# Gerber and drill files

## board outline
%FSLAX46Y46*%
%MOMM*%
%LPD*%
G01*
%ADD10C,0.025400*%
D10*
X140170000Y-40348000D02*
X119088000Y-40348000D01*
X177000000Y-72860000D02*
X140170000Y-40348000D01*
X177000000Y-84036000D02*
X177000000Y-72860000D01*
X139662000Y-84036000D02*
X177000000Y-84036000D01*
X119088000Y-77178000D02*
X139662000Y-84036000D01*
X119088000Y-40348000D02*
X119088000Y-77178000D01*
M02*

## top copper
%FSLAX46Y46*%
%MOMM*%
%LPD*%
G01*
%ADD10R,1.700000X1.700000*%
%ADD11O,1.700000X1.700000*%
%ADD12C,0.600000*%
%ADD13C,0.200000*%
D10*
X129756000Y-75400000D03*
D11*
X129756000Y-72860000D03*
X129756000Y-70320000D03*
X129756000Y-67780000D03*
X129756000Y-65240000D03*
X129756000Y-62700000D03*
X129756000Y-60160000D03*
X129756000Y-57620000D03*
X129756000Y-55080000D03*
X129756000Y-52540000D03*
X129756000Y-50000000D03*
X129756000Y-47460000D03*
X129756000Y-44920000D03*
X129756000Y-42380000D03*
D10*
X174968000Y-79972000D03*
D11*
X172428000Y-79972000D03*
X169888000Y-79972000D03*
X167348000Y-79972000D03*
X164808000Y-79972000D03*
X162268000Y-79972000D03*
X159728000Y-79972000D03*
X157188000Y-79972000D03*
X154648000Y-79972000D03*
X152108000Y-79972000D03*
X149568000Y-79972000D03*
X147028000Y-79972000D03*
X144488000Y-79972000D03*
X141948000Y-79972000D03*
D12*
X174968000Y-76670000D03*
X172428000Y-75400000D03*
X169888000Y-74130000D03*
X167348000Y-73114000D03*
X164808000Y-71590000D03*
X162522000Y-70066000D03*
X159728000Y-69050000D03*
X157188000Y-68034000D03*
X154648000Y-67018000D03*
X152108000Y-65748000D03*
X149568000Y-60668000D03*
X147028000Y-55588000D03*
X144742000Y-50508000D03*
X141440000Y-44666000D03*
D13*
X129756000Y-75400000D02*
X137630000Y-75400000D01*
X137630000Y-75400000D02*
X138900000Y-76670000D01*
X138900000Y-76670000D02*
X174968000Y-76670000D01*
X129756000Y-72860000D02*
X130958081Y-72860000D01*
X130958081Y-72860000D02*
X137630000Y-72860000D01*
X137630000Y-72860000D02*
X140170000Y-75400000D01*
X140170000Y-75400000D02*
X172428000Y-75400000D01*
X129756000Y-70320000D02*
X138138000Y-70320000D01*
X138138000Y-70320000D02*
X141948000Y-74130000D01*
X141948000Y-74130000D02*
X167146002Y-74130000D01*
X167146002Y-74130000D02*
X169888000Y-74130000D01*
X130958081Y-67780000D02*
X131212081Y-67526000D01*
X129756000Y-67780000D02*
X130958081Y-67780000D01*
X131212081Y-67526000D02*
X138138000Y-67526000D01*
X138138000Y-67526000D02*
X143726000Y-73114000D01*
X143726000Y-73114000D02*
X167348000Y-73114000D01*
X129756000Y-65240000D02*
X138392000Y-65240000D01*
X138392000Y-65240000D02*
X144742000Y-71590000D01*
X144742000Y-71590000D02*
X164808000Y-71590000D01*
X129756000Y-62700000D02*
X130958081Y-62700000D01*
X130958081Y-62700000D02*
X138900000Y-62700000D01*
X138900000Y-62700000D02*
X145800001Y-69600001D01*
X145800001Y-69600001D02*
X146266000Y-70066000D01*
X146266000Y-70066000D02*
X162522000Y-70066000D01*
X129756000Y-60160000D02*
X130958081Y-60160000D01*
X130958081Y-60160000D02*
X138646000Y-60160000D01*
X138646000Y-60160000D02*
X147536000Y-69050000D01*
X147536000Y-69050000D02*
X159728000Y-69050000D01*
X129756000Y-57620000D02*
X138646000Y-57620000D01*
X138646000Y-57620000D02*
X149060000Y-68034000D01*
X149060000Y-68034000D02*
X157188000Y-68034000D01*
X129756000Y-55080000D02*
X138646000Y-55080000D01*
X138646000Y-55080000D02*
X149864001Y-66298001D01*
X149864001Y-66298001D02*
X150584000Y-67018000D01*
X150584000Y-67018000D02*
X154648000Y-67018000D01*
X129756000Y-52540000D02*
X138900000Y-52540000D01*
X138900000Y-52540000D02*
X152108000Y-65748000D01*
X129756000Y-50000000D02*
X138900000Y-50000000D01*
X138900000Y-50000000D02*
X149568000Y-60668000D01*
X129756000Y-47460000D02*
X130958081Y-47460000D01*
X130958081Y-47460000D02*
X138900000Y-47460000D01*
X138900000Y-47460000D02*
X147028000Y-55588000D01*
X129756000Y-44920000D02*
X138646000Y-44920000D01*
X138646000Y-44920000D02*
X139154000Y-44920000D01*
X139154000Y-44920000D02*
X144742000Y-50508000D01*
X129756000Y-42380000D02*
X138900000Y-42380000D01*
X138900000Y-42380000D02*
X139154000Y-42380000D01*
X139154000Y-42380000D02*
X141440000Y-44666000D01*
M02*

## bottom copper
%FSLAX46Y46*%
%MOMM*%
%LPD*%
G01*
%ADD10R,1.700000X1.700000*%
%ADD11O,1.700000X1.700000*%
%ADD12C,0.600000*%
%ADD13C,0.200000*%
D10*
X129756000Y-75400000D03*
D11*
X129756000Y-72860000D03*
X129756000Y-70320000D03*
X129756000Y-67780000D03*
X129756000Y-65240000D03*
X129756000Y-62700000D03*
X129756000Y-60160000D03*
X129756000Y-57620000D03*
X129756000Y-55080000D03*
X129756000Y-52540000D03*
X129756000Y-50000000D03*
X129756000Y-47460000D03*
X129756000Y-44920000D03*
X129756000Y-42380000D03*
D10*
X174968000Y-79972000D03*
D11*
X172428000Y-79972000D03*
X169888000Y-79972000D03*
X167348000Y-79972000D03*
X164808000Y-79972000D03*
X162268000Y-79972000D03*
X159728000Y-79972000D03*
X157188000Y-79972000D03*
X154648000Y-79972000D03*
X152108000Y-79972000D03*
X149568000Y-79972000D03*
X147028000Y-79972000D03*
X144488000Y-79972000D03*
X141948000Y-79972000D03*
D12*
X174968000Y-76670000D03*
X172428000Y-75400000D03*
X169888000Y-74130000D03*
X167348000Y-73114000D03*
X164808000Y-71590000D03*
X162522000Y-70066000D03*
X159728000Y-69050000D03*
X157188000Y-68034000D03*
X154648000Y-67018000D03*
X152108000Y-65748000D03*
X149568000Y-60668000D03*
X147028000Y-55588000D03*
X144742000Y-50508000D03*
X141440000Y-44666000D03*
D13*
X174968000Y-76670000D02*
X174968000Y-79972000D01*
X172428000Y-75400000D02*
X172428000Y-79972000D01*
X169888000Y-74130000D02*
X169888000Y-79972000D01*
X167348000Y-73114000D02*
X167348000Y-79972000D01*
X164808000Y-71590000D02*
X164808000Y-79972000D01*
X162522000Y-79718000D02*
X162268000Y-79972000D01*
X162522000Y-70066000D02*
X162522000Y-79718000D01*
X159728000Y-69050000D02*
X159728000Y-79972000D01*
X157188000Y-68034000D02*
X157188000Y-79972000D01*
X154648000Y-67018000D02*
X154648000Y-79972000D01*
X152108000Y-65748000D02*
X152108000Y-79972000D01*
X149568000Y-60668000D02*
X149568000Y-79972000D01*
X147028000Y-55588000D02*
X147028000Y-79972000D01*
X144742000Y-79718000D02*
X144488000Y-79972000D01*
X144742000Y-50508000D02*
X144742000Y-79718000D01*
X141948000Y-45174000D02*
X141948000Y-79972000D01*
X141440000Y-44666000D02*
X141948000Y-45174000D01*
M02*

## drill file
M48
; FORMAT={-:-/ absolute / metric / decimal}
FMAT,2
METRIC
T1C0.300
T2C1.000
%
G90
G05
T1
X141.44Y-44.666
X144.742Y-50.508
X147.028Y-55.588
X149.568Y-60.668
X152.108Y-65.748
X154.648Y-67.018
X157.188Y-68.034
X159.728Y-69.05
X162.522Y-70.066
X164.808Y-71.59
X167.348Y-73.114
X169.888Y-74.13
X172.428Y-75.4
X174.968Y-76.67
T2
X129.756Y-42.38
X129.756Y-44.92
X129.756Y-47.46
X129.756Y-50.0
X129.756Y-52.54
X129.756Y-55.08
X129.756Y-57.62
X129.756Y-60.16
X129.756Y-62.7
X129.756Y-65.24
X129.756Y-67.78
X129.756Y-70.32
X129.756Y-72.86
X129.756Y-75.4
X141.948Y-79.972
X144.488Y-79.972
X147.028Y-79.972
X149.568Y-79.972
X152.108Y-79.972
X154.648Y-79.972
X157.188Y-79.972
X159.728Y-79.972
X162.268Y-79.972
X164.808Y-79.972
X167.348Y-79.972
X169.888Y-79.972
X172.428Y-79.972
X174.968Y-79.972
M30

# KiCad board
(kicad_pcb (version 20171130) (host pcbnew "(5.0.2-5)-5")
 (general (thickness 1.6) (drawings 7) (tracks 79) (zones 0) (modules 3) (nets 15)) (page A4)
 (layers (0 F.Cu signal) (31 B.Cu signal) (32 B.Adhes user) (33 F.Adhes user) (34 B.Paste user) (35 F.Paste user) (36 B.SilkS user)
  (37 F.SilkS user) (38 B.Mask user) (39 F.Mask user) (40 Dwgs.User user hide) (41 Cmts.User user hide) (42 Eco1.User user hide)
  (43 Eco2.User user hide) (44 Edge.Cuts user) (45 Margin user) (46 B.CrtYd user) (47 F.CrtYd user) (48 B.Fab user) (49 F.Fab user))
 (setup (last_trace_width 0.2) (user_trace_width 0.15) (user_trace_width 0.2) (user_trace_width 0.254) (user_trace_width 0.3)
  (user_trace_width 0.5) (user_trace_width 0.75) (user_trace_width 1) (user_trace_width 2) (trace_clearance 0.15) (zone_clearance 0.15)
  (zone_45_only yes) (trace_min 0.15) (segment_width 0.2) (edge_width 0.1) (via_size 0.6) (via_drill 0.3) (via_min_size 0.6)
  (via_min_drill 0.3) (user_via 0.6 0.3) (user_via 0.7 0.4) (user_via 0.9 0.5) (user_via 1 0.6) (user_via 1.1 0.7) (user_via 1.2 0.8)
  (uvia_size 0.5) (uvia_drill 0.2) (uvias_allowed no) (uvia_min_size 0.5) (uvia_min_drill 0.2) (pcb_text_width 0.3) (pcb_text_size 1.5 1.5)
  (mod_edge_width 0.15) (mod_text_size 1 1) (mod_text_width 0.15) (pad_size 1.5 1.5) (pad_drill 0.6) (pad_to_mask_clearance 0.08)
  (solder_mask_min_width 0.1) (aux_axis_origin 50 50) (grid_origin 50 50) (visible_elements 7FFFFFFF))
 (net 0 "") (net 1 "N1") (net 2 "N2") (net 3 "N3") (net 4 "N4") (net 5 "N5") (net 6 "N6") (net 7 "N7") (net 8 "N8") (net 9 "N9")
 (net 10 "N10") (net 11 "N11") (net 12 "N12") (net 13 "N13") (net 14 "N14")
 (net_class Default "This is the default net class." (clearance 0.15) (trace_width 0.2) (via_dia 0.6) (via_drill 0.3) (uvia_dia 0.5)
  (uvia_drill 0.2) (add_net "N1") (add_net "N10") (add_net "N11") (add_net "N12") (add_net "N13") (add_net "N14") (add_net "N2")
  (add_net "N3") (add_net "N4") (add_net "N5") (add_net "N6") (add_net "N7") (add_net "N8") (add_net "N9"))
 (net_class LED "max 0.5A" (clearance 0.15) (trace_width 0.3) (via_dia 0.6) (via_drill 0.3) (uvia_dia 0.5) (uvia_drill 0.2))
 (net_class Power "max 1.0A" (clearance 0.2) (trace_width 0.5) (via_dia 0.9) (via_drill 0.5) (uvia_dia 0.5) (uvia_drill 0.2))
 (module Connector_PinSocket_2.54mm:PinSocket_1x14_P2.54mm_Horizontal (layer B.Cu) (at 129.756 75.4)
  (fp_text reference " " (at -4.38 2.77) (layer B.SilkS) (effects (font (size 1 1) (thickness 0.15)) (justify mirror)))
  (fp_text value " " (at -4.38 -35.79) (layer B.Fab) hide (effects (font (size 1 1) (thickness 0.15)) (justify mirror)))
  (pad 1 thru_hole rect (at 0 0) (size 1.7 1.7) (drill 1) (layers *.Cu *.Mask) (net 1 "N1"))
  (pad 2 thru_hole oval (at 0 -2.54) (size 1.7 1.7) (drill 1) (layers *.Cu *.Mask) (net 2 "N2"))
  (pad 3 thru_hole oval (at 0 -5.08) (size 1.7 1.7) (drill 1) (layers *.Cu *.Mask) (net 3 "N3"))
  (pad 4 thru_hole oval (at 0 -7.62) (size 1.7 1.7) (drill 1) (layers *.Cu *.Mask) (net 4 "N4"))
  (pad 5 thru_hole oval (at 0 -10.16) (size 1.7 1.7) (drill 1) (layers *.Cu *.Mask) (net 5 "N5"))
  (pad 6 thru_hole oval (at 0 -12.7) (size 1.7 1.7) (drill 1) (layers *.Cu *.Mask) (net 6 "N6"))
  (pad 7 thru_hole oval (at 0 -15.24) (size 1.7 1.7) (drill 1) (layers *.Cu *.Mask) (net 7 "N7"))
  (pad 8 thru_hole oval (at 0 -17.78) (size 1.7 1.7) (drill 1) (layers *.Cu *.Mask) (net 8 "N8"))
  (pad 9 thru_hole oval (at 0 -20.32) (size 1.7 1.7) (drill 1) (layers *.Cu *.Mask) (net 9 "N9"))
  (pad 10 thru_hole oval (at 0 -22.86) (size 1.7 1.7) (drill 1) (layers *.Cu *.Mask) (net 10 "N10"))
  (pad 11 thru_hole oval (at 0 -25.4) (size 1.7 1.7) (drill 1) (layers *.Cu *.Mask) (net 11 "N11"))
  (pad 12 thru_hole oval (at 0 -27.94) (size 1.7 1.7) (drill 1) (layers *.Cu *.Mask) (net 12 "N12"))
  (pad 13 thru_hole oval (at 0 -30.48) (size 1.7 1.7) (drill 1) (layers *.Cu *.Mask) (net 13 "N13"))
  (pad 14 thru_hole oval (at 0 -33.02) (size 1.7 1.7) (drill 1) (layers *.Cu *.Mask) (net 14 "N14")))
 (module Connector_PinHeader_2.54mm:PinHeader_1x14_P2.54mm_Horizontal (layer F.Cu) (at 174.968 79.972 270)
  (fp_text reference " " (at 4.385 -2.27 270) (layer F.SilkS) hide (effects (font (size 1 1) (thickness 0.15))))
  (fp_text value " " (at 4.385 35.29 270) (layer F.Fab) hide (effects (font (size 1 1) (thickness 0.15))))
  (pad 1 thru_hole rect (at 0 0 270) (size 1.7 1.7) (drill 1) (layers *.Cu *.Mask) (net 1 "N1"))
  (pad 2 thru_hole oval (at 0 2.54 270) (size 1.7 1.7) (drill 1) (layers *.Cu *.Mask) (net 2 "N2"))
  (pad 3 thru_hole oval (at 0 5.08 270) (size 1.7 1.7) (drill 1) (layers *.Cu *.Mask) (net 3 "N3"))
  (pad 4 thru_hole oval (at 0 7.62 270) (size 1.7 1.7) (drill 1) (layers *.Cu *.Mask) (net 4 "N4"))
  (pad 5 thru_hole oval (at 0 10.16 270) (size 1.7 1.7) (drill 1) (layers *.Cu *.Mask) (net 5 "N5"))
  (pad 6 thru_hole oval (at 0 12.7 270) (size 1.7 1.7) (drill 1) (layers *.Cu *.Mask) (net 6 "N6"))
  (pad 7 thru_hole oval (at 0 15.24 270) (size 1.7 1.7) (drill 1) (layers *.Cu *.Mask) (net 7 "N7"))
  (pad 8 thru_hole oval (at 0 17.78 270) (size 1.7 1.7) (drill 1) (layers *.Cu *.Mask) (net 8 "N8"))
  (pad 9 thru_hole oval (at 0 20.32 270) (size 1.7 1.7) (drill 1) (layers *.Cu *.Mask) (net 9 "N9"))
  (pad 10 thru_hole oval (at 0 22.86 270) (size 1.7 1.7) (drill 1) (layers *.Cu *.Mask) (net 10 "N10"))
  (pad 11 thru_hole oval (at 0 25.4 270) (size 1.7 1.7) (drill 1) (layers *.Cu *.Mask) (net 11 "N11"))
  (pad 12 thru_hole oval (at 0 27.94 270) (size 1.7 1.7) (drill 1) (layers *.Cu *.Mask) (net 12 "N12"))
  (pad 13 thru_hole oval (at 0 30.48 270) (size 1.7 1.7) (drill 1) (layers *.Cu *.Mask) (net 13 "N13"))
  (pad 14 thru_hole oval (at 0 33.02 270) (size 1.7 1.7) (drill 1) (layers *.Cu *.Mask) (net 14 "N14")))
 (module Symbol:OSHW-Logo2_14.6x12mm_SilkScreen (layer B.Cu) (at 152.108 66.256 180)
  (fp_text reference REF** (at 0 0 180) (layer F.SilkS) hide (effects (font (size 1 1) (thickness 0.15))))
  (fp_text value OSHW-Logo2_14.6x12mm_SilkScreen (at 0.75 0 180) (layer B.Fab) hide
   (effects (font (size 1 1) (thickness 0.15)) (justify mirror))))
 (gr_line (start 140.17 40.348) (end 119.088 40.348) (layer Edge.Cuts) (width 0.0254))
 (gr_line (start 177 72.86) (end 140.17 40.348) (layer Edge.Cuts) (width 0.0254))
 (gr_line (start 177 84.036) (end 177 72.86) (layer Edge.Cuts) (width 0.0254))
 (gr_line (start 139.662 84.036) (end 177 84.036) (layer Edge.Cuts) (width 0.0254))
 (gr_line (start 119.088 77.178) (end 139.662 84.036) (layer Edge.Cuts) (width 0.0254))
 (gr_line (start 119.088 40.348) (end 119.088 77.178) (layer Edge.Cuts) (width 0.0254))
 (segment (start 129.756 75.4) (end 137.63 75.4) (width 0.2) (layer F.Cu) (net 1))
 (segment (start 137.63 75.4) (end 138.9 76.67) (width 0.2) (layer F.Cu) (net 1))
 (segment (start 138.9 76.67) (end 174.968 76.67) (width 0.2) (layer F.Cu) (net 1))
 (via (at 174.968 76.67) (size 0.6) (drill 0.3) (layers F.Cu B.Cu) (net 1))
 (segment (start 174.968 76.67) (end 174.968 79.972) (width 0.2) (layer B.Cu) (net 1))
 (segment (start 129.756 72.86) (end 130.958081 72.86) (width 0.2) (layer F.Cu) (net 2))
 (segment (start 130.958081 72.86) (end 137.63 72.86) (width 0.2) (layer F.Cu) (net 2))
 (segment (start 137.63 72.86) (end 140.17 75.4) (width 0.2) (layer F.Cu) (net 2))
 (segment (start 140.17 75.4) (end 172.428 75.4) (width 0.2) (layer F.Cu) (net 2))
 (via (at 172.428 75.4) (size 0.6) (drill 0.3) (layers F.Cu B.Cu) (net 2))
 (segment (start 172.428 75.4) (end 172.428 79.972) (width 0.2) (layer B.Cu) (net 2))
 (segment (start 129.756 70.32) (end 138.138 70.32) (width 0.2) (layer F.Cu) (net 3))
 (segment (start 138.138 70.32) (end 141.948 74.13) (width 0.2) (layer F.Cu) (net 3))
 (segment (start 141.948 74.13) (end 167.146002 74.13) (width 0.2) (layer F.Cu) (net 3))
 (via (at 169.888 74.13) (size 0.6) (drill 0.3) (layers F.Cu B.Cu) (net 3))
 (segment (start 167.146002 74.13) (end 169.888 74.13) (width 0.2) (layer F.Cu) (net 3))
 (segment (start 169.888 74.13) (end 169.888 79.972) (width 0.2) (layer B.Cu) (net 3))
 (segment (start 130.958081 67.78) (end 131.212081 67.526) (width 0.2) (layer F.Cu) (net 4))
 (segment (start 129.756 67.78) (end 130.958081 67.78) (width 0.2) (layer F.Cu) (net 4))
 (segment (start 131.212081 67.526) (end 138.138 67.526) (width 0.2) (layer F.Cu) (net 4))
 (segment (start 138.138 67.526) (end 143.726 73.114) (width 0.2) (layer F.Cu) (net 4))
 (via (at 167.348 73.114) (size 0.6) (drill 0.3) (layers F.Cu B.Cu) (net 4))
 (segment (start 143.726 73.114) (end 167.348 73.114) (width 0.2) (layer F.Cu) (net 4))
 (segment (start 167.348 73.114) (end 167.348 79.972) (width 0.2) (layer B.Cu) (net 4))
 (segment (start 129.756 65.24) (end 138.392 65.24) (width 0.2) (layer F.Cu) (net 5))
 (segment (start 138.392 65.24) (end 144.742 71.59) (width 0.2) (layer F.Cu) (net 5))
 (segment (start 144.742 71.59) (end 164.808 71.59) (width 0.2) (layer F.Cu) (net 5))
 (via (at 164.808 71.59) (size 0.6) (drill 0.3) (layers F.Cu B.Cu) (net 5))
 (segment (start 164.808 71.59) (end 164.808 79.972) (width 0.2) (layer B.Cu) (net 5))
 (segment (start 129.756 62.7) (end 130.958081 62.7) (width 0.2) (layer F.Cu) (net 6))
 (segment (start 130.958081 62.7) (end 138.9 62.7) (width 0.2) (layer F.Cu) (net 6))
 (segment (start 138.9 62.7) (end 145.800001 69.600001) (width 0.2) (layer F.Cu) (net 6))
 (segment (start 145.800001 69.600001) (end 146.266 70.066) (width 0.2) (layer F.Cu) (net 6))
 (via (at 162.522 70.066) (size 0.6) (drill 0.3) (layers F.Cu B.Cu) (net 6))
 (segment (start 146.266 70.066) (end 162.522 70.066) (width 0.2) (layer F.Cu) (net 6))
 (segment (start 162.522 79.718) (end 162.268 79.972) (width 0.2) (layer B.Cu) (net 6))
 (segment (start 162.522 70.066) (end 162.522 79.718) (width 0.2) (layer B.Cu) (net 6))
 (segment (start 129.756 60.16) (end 130.958081 60.16) (width 0.2) (layer F.Cu) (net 7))
 (segment (start 130.958081 60.16) (end 138.646 60.16) (width 0.2) (layer F.Cu) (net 7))
 (segment (start 138.646 60.16) (end 147.536 69.05) (width 0.2) (layer F.Cu) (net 7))
 (via (at 159.728 69.05) (size 0.6) (drill 0.3) (layers F.Cu B.Cu) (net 7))
 (segment (start 147.536 69.05) (end 159.728 69.05) (width 0.2) (layer F.Cu) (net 7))
 (segment (start 159.728 69.05) (end 159.728 79.972) (width 0.2) (layer B.Cu) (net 7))
 (segment (start 129.756 57.62) (end 138.646 57.62) (width 0.2) (layer F.Cu) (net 8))
 (segment (start 138.646 57.62) (end 149.06 68.034) (width 0.2) (layer F.Cu) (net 8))
 (segment (start 149.06 68.034) (end 157.188 68.034) (width 0.2) (layer F.Cu) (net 8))
 (via (at 157.188 68.034) (size 0.6) (drill 0.3) (layers F.Cu B.Cu) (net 8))
 (segment (start 157.188 68.034) (end 157.188 79.972) (width 0.2) (layer B.Cu) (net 8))
 (segment (start 129.756 55.08) (end 138.646 55.08) (width 0.2) (layer F.Cu) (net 9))
 (segment (start 138.646 55.08) (end 149.864001 66.298001) (width 0.2) (layer F.Cu) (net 9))
 (segment (start 149.864001 66.298001) (end 150.584 67.018) (width 0.2) (layer F.Cu) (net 9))
 (segment (start 150.584 67.018) (end 154.648 67.018) (width 0.2) (layer F.Cu) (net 9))
 (via (at 154.648 67.018) (size 0.6) (drill 0.3) (layers F.Cu B.Cu) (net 9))
 (segment (start 154.648 67.018) (end 154.648 79.972) (width 0.2) (layer B.Cu) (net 9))
 (segment (start 129.756 52.54) (end 138.9 52.54) (width 0.2) (layer F.Cu) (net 10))
 (segment (start 138.9 52.54) (end 152.108 65.748) (width 0.2) (layer F.Cu) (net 10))
 (via (at 152.108 65.748) (size 0.6) (drill 0.3) (layers F.Cu B.Cu) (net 10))
 (segment (start 152.108 65.748) (end 152.108 79.972) (width 0.2) (layer B.Cu) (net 10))
 (segment (start 129.756 50) (end 138.9 50) (width 0.2) (layer F.Cu) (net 11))
 (segment (start 138.9 50) (end 149.568 60.668) (width 0.2) (layer F.Cu) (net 11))
 (via (at 149.568 60.668) (size 0.6) (drill 0.3) (layers F.Cu B.Cu) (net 11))
 (segment (start 149.568 60.668) (end 149.568 79.972) (width 0.2) (layer B.Cu) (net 11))
 (segment (start 129.756 47.46) (end 130.958081 47.46) (width 0.2) (layer F.Cu) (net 12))
 (segment (start 130.958081 47.46) (end 138.9 47.46) (width 0.2) (layer F.Cu) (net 12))
 (via (at 147.028 55.588) (size 0.6) (drill 0.3) (layers F.Cu B.Cu) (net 12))
 (segment (start 138.9 47.46) (end 147.028 55.588) (width 0.2) (layer F.Cu) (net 12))
 (segment (start 147.028 55.588) (end 147.028 79.972) (width 0.2) (layer B.Cu) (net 12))
 (segment (start 129.756 44.92) (end 138.646 44.92) (width 0.2) (layer F.Cu) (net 13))
 (segment (start 138.646 44.92) (end 139.154 44.92) (width 0.2) (layer F.Cu) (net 13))
 (via (at 144.742 50.508) (size 0.6) (drill 0.3) (layers F.Cu B.Cu) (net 13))
 (segment (start 139.154 44.92) (end 144.742 50.508) (width 0.2) (layer F.Cu) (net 13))
 (segment (start 144.742 79.718) (end 144.488 79.972) (width 0.2) (layer B.Cu) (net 13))
 (segment (start 144.742 50.508) (end 144.742 79.718) (width 0.2) (layer B.Cu) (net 13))
 (segment (start 129.756 42.38) (end 138.9 42.38) (width 0.2) (layer F.Cu) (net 14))
 (segment (start 138.9 42.38) (end 139.154 42.38) (width 0.2) (layer F.Cu) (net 14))
 (via (at 141.44 44.666) (size 0.6) (drill 0.3) (layers F.Cu B.Cu) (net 14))
 (segment (start 139.154 42.38) (end 141.44 44.666) (width 0.2) (layer F.Cu) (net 14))
 (segment (start 141.948 45.174) (end 141.948 79.972) (width 0.2) (layer B.Cu) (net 14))
 (segment (start 141.44 44.666) (end 141.948 45.174) (width 0.2) (layer B.Cu) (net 14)))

